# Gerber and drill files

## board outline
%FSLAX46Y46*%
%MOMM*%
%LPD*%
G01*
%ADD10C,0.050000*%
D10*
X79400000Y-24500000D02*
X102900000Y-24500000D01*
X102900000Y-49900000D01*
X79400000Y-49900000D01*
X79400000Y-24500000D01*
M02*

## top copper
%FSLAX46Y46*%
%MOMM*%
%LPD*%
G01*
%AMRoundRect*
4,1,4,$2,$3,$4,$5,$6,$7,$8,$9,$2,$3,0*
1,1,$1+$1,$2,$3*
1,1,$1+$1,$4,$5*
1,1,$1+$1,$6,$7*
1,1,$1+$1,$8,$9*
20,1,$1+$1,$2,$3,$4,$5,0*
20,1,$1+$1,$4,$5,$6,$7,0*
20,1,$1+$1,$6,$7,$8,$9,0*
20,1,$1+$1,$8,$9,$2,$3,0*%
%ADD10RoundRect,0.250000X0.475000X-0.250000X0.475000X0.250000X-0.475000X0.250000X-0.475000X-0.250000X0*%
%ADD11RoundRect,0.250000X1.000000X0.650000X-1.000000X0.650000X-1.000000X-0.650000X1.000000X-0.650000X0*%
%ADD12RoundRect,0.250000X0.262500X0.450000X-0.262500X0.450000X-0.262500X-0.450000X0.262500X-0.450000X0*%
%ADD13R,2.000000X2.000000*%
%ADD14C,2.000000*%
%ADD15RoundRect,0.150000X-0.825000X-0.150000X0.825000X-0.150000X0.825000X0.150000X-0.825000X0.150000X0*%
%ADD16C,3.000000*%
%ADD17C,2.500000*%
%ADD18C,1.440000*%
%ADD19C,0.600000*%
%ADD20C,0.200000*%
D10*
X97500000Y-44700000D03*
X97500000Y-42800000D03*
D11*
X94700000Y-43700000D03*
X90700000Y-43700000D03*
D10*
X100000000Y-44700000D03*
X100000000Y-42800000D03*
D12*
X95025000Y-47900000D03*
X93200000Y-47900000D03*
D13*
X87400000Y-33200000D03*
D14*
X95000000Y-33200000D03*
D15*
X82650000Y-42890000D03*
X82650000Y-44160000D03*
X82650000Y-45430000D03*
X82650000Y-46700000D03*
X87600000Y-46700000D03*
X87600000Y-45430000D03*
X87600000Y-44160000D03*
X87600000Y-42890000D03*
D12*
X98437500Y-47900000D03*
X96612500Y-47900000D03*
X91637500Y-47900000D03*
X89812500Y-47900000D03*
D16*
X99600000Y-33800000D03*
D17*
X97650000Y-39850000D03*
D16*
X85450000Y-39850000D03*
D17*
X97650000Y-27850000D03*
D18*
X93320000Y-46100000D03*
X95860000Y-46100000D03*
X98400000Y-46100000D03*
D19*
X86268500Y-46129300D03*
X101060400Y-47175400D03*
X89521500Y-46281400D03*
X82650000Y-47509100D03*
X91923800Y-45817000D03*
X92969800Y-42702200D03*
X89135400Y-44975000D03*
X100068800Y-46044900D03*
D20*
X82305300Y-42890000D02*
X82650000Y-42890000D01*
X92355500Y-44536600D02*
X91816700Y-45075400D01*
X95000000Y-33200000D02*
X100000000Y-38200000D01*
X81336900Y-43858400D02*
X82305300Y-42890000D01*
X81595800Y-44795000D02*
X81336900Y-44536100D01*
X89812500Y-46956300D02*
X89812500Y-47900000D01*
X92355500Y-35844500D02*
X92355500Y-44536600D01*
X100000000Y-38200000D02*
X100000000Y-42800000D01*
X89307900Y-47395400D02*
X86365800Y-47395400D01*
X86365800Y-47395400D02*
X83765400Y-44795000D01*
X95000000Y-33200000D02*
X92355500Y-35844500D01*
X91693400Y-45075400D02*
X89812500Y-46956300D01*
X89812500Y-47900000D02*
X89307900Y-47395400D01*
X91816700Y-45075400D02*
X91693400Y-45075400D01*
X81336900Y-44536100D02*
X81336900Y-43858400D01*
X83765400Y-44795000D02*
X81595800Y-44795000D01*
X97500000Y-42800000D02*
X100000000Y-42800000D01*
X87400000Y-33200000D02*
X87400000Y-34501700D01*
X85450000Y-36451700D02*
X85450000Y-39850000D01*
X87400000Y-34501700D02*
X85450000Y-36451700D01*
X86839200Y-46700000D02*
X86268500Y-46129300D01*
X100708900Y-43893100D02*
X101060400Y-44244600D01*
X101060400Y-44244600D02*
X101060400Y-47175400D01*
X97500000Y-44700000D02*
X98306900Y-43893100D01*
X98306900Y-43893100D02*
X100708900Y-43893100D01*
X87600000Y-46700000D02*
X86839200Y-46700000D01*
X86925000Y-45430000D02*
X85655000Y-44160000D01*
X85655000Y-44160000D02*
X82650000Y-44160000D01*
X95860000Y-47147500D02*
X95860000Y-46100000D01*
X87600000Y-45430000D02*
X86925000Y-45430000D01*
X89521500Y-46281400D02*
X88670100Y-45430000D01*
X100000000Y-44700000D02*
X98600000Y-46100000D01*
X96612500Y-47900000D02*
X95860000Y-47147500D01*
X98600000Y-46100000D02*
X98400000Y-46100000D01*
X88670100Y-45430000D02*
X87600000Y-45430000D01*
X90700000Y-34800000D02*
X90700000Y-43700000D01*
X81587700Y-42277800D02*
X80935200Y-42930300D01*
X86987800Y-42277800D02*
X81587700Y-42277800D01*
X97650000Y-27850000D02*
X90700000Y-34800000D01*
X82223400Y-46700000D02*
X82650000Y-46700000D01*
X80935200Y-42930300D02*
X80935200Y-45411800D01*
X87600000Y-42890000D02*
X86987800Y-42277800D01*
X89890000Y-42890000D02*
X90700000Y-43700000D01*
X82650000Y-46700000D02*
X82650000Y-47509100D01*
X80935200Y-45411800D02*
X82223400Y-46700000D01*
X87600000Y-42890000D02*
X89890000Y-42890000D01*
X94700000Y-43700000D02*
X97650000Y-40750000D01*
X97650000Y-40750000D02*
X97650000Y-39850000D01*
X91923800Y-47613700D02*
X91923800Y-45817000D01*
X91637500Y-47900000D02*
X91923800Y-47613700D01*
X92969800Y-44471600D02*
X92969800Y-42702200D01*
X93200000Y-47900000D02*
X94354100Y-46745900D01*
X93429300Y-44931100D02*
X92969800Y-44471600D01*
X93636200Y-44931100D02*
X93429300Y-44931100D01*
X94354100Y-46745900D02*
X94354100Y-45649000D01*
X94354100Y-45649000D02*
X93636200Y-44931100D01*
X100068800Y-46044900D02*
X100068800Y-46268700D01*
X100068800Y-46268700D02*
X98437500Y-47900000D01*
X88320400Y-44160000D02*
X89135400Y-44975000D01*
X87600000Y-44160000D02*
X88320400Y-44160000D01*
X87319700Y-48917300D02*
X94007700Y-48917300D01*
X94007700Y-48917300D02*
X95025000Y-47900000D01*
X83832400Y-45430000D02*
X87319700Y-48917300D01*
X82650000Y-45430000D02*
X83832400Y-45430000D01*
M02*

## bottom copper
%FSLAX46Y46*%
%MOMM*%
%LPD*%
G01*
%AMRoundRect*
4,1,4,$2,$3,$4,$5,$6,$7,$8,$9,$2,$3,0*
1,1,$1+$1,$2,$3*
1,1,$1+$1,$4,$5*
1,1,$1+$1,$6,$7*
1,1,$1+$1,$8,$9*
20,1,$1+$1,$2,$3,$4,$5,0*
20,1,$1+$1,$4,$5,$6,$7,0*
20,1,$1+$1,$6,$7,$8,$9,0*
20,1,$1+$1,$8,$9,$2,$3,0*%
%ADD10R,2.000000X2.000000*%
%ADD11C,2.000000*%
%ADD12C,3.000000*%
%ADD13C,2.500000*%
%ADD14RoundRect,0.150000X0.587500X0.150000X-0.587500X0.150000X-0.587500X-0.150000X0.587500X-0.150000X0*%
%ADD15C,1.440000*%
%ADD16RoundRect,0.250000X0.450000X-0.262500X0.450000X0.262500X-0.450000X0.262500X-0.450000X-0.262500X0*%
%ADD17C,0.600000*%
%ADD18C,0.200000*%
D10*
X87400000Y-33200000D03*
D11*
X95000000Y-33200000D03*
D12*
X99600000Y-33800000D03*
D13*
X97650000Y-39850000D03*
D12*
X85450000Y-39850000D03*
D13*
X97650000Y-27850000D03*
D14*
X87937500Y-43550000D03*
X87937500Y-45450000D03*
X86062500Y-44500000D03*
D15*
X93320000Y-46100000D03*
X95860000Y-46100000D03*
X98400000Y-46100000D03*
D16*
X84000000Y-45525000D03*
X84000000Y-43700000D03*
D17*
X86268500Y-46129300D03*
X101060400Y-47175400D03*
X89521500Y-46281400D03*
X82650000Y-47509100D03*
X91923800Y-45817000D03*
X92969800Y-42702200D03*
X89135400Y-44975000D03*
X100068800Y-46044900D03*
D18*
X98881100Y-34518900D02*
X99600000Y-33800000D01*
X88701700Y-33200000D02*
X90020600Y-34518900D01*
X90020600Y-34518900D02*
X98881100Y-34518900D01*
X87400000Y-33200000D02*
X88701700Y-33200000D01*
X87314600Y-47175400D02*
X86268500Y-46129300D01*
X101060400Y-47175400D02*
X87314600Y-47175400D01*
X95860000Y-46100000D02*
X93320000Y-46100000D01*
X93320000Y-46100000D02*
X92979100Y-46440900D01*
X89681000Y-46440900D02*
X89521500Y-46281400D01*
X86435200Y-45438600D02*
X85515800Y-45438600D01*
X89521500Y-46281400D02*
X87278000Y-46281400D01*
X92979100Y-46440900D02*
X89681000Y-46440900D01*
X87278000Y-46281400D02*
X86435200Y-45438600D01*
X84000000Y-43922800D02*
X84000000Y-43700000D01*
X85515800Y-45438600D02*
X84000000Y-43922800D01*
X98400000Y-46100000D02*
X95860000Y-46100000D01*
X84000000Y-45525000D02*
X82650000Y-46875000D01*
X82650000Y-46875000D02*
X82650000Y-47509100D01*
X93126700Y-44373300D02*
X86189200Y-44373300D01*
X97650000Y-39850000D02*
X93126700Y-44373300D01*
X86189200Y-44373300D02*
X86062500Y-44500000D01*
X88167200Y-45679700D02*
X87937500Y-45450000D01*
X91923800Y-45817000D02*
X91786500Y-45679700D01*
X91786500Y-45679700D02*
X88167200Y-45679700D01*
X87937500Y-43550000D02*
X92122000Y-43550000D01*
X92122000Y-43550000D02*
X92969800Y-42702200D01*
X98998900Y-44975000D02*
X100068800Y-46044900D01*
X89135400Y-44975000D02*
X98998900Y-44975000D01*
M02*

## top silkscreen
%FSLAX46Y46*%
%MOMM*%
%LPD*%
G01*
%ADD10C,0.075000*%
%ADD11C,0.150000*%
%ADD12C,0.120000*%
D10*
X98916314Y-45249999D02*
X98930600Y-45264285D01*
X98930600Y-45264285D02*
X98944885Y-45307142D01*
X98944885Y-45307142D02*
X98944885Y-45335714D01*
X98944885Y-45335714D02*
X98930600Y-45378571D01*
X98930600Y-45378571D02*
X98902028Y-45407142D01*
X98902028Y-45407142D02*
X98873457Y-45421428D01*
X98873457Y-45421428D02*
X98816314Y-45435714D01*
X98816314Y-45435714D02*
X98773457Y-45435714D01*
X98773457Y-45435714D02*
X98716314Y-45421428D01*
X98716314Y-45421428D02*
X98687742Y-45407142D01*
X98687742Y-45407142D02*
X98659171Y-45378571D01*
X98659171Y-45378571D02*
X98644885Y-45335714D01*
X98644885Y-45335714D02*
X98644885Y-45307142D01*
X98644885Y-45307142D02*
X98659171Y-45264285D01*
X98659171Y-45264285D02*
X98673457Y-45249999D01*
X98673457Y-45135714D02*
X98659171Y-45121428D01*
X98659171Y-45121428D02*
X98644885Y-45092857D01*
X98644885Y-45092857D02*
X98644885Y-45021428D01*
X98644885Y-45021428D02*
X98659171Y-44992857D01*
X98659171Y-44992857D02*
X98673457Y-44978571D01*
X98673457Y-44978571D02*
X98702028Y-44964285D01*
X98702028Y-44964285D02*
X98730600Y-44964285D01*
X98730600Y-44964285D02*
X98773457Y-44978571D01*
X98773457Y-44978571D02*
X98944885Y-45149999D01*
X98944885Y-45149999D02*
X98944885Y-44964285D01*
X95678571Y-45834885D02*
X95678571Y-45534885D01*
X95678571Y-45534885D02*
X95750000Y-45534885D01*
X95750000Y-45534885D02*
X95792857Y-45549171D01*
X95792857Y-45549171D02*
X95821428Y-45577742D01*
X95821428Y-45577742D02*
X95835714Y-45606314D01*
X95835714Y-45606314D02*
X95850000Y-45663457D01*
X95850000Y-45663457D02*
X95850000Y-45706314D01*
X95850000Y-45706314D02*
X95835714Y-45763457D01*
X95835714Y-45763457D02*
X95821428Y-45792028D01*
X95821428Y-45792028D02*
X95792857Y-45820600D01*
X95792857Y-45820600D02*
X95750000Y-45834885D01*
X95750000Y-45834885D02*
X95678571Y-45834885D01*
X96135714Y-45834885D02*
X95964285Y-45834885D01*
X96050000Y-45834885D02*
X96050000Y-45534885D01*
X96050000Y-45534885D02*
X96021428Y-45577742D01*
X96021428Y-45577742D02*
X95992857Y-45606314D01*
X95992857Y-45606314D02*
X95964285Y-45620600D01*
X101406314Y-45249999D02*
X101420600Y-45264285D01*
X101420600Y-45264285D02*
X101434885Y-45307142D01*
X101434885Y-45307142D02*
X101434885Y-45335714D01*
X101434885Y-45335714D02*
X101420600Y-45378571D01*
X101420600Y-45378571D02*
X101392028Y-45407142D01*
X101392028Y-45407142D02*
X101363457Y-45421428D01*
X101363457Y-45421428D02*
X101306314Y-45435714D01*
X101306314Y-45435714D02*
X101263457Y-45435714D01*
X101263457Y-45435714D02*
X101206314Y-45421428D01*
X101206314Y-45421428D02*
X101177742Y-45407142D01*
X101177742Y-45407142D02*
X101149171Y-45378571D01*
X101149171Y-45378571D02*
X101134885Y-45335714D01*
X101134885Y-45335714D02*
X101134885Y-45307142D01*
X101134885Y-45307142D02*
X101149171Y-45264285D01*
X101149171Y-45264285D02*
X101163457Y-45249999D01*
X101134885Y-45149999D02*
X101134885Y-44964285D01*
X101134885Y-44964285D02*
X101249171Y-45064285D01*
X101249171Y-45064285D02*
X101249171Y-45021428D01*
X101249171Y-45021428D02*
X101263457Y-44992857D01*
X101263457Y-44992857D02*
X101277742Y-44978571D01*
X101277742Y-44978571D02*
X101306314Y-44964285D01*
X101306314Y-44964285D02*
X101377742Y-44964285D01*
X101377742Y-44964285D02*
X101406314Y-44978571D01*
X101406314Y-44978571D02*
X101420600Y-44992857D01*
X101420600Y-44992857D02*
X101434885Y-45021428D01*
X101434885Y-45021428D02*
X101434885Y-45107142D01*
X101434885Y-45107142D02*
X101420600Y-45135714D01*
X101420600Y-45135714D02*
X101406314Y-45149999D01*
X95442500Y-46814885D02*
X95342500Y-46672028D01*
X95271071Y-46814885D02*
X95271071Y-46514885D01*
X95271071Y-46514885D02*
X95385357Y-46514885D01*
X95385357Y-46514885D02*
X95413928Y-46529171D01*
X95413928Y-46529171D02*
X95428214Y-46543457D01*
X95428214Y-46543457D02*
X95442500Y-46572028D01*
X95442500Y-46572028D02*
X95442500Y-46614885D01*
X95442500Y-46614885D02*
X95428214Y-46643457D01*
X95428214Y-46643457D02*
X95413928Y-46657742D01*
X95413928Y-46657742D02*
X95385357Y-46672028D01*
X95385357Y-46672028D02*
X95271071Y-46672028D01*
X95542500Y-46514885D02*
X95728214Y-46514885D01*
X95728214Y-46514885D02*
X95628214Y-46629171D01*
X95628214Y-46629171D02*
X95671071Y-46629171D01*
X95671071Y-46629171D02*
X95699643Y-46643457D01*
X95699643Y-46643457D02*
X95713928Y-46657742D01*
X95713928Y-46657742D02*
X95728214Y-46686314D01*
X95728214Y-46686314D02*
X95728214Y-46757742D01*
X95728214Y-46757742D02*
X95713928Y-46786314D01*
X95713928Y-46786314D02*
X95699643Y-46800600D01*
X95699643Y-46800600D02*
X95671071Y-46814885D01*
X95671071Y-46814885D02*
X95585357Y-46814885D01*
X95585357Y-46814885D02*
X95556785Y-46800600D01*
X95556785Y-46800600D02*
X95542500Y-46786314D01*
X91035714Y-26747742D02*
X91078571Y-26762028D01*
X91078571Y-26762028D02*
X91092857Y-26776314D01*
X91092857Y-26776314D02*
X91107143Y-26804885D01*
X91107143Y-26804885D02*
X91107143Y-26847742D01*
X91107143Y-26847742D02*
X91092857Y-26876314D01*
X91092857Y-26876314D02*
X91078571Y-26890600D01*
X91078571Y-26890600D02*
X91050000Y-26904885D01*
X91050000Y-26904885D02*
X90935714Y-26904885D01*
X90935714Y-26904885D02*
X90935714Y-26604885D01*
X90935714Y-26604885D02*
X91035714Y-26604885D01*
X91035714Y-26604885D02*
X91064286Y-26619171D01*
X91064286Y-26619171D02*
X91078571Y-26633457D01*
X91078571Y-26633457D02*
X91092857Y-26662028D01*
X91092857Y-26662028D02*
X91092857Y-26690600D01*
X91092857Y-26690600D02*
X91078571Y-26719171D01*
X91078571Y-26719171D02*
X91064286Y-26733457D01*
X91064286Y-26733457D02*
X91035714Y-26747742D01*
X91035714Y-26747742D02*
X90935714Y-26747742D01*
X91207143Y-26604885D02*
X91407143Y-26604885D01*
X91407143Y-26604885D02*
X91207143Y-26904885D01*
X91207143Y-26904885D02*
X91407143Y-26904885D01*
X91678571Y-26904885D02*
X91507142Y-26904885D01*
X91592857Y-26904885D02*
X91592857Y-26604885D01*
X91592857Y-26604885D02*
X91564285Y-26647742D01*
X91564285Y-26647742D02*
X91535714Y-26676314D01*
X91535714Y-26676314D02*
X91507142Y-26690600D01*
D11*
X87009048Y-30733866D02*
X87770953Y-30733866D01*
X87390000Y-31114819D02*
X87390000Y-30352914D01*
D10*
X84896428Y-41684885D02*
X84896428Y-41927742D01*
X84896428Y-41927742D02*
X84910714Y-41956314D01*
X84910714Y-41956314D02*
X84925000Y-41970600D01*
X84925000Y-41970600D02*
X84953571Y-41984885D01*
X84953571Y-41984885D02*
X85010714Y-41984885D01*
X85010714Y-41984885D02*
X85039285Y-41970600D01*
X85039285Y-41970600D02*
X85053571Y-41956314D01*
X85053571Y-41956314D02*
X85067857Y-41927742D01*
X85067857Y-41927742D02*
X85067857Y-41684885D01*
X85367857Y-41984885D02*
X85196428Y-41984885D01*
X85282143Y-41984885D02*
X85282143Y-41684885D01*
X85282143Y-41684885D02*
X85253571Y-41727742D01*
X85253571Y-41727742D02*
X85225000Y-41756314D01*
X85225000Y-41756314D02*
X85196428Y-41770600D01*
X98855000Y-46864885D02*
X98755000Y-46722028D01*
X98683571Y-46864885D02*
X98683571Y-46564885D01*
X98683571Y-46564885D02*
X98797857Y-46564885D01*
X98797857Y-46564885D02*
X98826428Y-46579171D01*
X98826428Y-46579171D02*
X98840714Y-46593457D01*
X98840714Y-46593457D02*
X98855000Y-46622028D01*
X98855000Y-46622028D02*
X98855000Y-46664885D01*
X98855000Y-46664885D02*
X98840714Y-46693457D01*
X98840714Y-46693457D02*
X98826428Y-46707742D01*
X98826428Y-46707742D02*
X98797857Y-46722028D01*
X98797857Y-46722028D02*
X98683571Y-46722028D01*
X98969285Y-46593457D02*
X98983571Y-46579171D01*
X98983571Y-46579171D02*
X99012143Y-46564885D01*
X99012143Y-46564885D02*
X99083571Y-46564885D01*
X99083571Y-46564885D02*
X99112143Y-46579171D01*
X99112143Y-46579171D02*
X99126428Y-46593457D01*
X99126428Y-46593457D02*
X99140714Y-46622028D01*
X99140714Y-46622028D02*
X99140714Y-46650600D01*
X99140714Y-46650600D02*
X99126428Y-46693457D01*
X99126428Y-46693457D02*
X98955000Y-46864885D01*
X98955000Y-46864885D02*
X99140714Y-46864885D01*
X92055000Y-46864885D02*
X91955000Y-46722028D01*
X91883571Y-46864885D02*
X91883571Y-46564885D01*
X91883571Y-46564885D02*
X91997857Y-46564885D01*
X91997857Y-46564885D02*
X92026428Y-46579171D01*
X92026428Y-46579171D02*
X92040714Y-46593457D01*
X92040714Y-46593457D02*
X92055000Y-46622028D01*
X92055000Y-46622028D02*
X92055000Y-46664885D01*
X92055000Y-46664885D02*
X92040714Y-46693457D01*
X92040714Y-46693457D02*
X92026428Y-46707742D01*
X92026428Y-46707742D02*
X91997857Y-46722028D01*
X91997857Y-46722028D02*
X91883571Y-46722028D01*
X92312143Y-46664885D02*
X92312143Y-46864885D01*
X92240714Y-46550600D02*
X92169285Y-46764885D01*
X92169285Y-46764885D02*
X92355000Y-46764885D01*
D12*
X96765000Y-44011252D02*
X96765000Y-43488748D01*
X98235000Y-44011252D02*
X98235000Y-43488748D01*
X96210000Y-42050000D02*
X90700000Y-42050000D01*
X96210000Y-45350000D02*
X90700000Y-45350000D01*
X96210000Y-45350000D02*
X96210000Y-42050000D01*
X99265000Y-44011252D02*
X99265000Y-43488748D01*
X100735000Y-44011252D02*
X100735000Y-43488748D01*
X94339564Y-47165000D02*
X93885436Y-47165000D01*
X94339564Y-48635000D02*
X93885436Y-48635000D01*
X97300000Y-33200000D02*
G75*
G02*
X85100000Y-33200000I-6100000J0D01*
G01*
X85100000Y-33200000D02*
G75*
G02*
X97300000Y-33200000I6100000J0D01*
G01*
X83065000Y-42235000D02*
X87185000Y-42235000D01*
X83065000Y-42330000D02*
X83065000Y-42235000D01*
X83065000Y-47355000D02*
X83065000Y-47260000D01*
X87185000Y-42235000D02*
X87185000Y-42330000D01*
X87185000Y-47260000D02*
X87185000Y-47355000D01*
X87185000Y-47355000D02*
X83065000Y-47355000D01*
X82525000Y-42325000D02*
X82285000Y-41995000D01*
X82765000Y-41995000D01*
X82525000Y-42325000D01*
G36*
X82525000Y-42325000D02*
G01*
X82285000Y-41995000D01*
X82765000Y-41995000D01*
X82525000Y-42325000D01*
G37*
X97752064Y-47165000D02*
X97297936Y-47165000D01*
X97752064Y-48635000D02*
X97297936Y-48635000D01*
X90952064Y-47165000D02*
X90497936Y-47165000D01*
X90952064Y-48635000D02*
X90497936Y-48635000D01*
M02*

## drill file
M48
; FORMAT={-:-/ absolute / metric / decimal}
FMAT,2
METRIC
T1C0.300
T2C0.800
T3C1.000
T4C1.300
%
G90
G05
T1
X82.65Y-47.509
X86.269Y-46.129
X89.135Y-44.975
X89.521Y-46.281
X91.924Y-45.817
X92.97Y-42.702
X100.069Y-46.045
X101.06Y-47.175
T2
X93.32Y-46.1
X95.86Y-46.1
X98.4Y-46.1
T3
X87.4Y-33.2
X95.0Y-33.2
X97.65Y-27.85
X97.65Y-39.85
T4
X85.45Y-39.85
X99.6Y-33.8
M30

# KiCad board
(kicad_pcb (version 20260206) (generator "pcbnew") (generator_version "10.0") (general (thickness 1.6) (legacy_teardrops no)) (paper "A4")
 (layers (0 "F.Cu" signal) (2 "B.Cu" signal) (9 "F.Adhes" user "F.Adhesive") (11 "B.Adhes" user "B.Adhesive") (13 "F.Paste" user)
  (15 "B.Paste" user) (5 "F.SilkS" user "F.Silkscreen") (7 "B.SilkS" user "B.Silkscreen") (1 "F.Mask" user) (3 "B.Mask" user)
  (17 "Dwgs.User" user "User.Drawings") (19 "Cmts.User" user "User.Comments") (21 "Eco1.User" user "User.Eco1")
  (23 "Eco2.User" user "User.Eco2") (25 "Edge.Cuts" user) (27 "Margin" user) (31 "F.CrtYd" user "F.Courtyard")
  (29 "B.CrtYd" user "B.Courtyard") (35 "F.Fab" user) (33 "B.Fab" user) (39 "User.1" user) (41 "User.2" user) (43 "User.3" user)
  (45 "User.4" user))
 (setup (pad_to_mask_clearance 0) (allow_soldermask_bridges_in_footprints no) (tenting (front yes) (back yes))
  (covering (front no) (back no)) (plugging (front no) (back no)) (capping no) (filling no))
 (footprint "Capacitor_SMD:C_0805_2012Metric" (layer "F.Cu") (at 97.5 43.75 90)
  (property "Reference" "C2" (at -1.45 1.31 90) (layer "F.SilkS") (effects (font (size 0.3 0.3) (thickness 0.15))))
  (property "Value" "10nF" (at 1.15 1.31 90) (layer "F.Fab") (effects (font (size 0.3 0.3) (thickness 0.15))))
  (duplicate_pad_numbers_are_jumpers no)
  (fp_line (start -0.261252 -0.735) (end 0.261252 -0.735) (stroke (width 0.12) (type solid)) (layer "F.SilkS"))
  (fp_line (start -0.261252 0.735) (end 0.261252 0.735) (stroke (width 0.12) (type solid)) (layer "F.SilkS"))
  (pad "1" smd roundrect (at -0.95 0 90) (size 1 1.45) (layers "F.Cu" "F.Mask" "F.Paste") (roundrect_rratio 0.25) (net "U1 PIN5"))
  (pad "2" smd roundrect (at 0.95 0 90) (size 1 1.45) (layers "F.Cu" "F.Mask" "F.Paste") (roundrect_rratio 0.25) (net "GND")))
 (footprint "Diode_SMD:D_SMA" (layer "F.Cu") (at 92.7 43.7 180)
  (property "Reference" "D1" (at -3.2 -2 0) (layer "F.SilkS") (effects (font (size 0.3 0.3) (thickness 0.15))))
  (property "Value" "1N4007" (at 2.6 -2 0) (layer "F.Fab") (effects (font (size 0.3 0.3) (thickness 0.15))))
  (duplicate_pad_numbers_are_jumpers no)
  (fp_line (start -3.51 1.65) (end 2 1.65) (stroke (width 0.12) (type solid)) (layer "F.SilkS"))
  (fp_line (start -3.51 -1.65) (end 2 -1.65) (stroke (width 0.12) (type solid)) (layer "F.SilkS"))
  (fp_line (start -3.51 -1.65) (end -3.51 1.65) (stroke (width 0.12) (type solid)) (layer "F.SilkS"))
  (pad "1" smd roundrect (at -2 0 180) (size 2.5 1.8) (layers "F.Cu" "F.Mask" "F.Paste") (roundrect_rratio 0.1388888889) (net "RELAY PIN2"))
  (pad "2" smd roundrect (at 2 0 180) (size 2.5 1.8) (layers "F.Cu" "F.Mask" "F.Paste") (roundrect_rratio 0.1388888889) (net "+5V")))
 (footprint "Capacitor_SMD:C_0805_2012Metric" (layer "F.Cu") (at 100 43.75 90)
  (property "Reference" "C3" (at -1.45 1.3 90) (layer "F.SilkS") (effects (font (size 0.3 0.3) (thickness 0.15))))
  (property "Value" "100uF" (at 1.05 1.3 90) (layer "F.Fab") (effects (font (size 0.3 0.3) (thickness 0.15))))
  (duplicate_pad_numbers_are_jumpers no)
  (fp_line (start -0.261252 -0.735) (end 0.261252 -0.735) (stroke (width 0.12) (type solid)) (layer "F.SilkS"))
  (fp_line (start -0.261252 0.735) (end 0.261252 0.735) (stroke (width 0.12) (type solid)) (layer "F.SilkS"))
  (pad "1" smd roundrect (at -0.95 0 90) (size 1 1.45) (layers "F.Cu" "F.Mask" "F.Paste") (roundrect_rratio 0.25) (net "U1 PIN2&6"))
  (pad "2" smd roundrect (at 0.95 0 90) (size 1 1.45) (layers "F.Cu" "F.Mask" "F.Paste") (roundrect_rratio 0.25) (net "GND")))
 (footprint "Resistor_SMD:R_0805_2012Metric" (layer "F.Cu") (at 94.1125 47.9 180)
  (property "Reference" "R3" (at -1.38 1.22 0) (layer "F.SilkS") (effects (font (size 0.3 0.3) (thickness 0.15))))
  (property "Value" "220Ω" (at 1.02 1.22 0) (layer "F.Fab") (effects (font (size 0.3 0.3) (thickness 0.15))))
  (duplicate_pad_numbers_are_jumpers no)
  (fp_line (start -0.227064 0.735) (end 0.227064 0.735) (stroke (width 0.12) (type solid)) (layer "F.SilkS"))
  (fp_line (start -0.227064 -0.735) (end 0.227064 -0.735) (stroke (width 0.12) (type solid)) (layer "F.SilkS"))
  (pad "1" smd roundrect (at -0.9125 0 180) (size 1.025 1.4) (layers "F.Cu" "F.Mask" "F.Paste") (roundrect_rratio 0.243902) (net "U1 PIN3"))
  (pad "2" smd roundrect (at 0.9125 0 180) (size 1.025 1.4) (layers "F.Cu" "F.Mask" "F.Paste") (roundrect_rratio 0.243902)
   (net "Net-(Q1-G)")))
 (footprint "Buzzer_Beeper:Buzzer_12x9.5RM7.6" (layer "F.Cu") (at 87.4 33.2)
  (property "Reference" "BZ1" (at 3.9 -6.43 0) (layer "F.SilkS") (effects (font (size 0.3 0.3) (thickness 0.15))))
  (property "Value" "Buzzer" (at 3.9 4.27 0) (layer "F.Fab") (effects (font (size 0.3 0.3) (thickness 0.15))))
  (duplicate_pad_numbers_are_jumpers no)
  (fp_circle (center 3.8 0) (end 9.9 0) (stroke (width 0.12) (type solid)) (fill no) (layer "F.SilkS"))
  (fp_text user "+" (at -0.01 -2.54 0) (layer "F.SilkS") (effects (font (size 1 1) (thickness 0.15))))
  (pad "1" thru_hole rect (at 0 0) (size 2 2) (drill 1) (layers "*.Cu" "*.Mask") (remove_unused_layers no) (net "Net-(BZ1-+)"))
  (pad "2" thru_hole circle (at 7.6 0) (size 2 2) (drill 1) (layers "*.Cu" "*.Mask") (remove_unused_layers no) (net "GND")))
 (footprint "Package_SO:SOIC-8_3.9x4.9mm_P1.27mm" (layer "F.Cu") (at 85.125 44.795)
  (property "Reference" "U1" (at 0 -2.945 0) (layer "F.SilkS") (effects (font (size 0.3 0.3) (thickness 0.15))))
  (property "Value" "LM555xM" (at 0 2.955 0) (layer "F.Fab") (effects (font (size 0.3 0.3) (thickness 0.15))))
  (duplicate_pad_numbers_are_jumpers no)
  (fp_line (start -2.06 -2.56) (end 2.06 -2.56) (stroke (width 0.12) (type solid)) (layer "F.SilkS"))
  (fp_line (start -2.06 -2.465) (end -2.06 -2.56) (stroke (width 0.12) (type solid)) (layer "F.SilkS"))
  (fp_line (start -2.06 2.56) (end -2.06 2.465) (stroke (width 0.12) (type solid)) (layer "F.SilkS"))
  (fp_line (start 2.06 -2.56) (end 2.06 -2.465) (stroke (width 0.12) (type solid)) (layer "F.SilkS"))
  (fp_line (start 2.06 2.465) (end 2.06 2.56) (stroke (width 0.12) (type solid)) (layer "F.SilkS"))
  (fp_line (start 2.06 2.56) (end -2.06 2.56) (stroke (width 0.12) (type solid)) (layer "F.SilkS"))
  (fp_poly (pts (xy -2.6 -2.47) (xy -2.84 -2.8) (xy -2.36 -2.8)) (stroke (width 0.12) (type solid)) (fill yes) (layer "F.SilkS"))
  (pad "1" smd roundrect (at -2.475 -1.905) (size 1.95 0.6) (layers "F.Cu" "F.Mask" "F.Paste") (roundrect_rratio 0.25) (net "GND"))
  (pad "2" smd roundrect (at -2.475 -0.635) (size 1.95 0.6) (layers "F.Cu" "F.Mask" "F.Paste") (roundrect_rratio 0.25) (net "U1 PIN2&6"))
  (pad "3" smd roundrect (at -2.475 0.635) (size 1.95 0.6) (layers "F.Cu" "F.Mask" "F.Paste") (roundrect_rratio 0.25) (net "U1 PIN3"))
  (pad "4" smd roundrect (at -2.475 1.905) (size 1.95 0.6) (layers "F.Cu" "F.Mask" "F.Paste") (roundrect_rratio 0.25) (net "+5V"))
  (pad "5" smd roundrect (at 2.475 1.905) (size 1.95 0.6) (layers "F.Cu" "F.Mask" "F.Paste") (roundrect_rratio 0.25) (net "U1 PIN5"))
  (pad "6" smd roundrect (at 2.475 0.635) (size 1.95 0.6) (layers "F.Cu" "F.Mask" "F.Paste") (roundrect_rratio 0.25) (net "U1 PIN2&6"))
  (pad "7" smd roundrect (at 2.475 -0.635) (size 1.95 0.6) (layers "F.Cu" "F.Mask" "F.Paste") (roundrect_rratio 0.25) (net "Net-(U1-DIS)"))
  (pad "8" smd roundrect (at 2.475 -1.905) (size 1.95 0.6) (layers "F.Cu" "F.Mask" "F.Paste") (roundrect_rratio 0.25) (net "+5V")))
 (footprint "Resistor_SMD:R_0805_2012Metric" (layer "F.Cu") (at 97.525 47.9 180)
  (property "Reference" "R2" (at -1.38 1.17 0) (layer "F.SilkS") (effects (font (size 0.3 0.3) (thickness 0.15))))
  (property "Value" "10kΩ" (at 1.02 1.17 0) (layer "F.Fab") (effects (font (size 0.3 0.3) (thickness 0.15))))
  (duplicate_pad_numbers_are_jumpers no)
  (fp_line (start -0.227064 0.735) (end 0.227064 0.735) (stroke (width 0.12) (type solid)) (layer "F.SilkS"))
  (fp_line (start -0.227064 -0.735) (end 0.227064 -0.735) (stroke (width 0.12) (type solid)) (layer "F.SilkS"))
  (pad "1" smd roundrect (at -0.9125 0 180) (size 1.025 1.4) (layers "F.Cu" "F.Mask" "F.Paste") (roundrect_rratio 0.243902)
   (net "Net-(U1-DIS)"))
  (pad "2" smd roundrect (at 0.9125 0 180) (size 1.025 1.4) (layers "F.Cu" "F.Mask" "F.Paste") (roundrect_rratio 0.243902) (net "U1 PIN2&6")))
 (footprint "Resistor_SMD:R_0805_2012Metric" (layer "F.Cu") (at 90.725 47.9 180)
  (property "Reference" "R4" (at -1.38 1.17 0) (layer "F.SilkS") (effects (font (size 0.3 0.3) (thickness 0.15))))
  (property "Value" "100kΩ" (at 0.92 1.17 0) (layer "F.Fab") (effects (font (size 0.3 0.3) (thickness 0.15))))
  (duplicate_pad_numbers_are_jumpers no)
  (fp_line (start -0.227064 0.735) (end 0.227064 0.735) (stroke (width 0.12) (type solid)) (layer "F.SilkS"))
  (fp_line (start -0.227064 -0.735) (end 0.227064 -0.735) (stroke (width 0.12) (type solid)) (layer "F.SilkS"))
  (pad "1" smd roundrect (at -0.9125 0 180) (size 1.025 1.4) (layers "F.Cu" "F.Mask" "F.Paste") (roundrect_rratio 0.243902)
   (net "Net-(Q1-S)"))
  (pad "2" smd roundrect (at 0.9125 0 180) (size 1.025 1.4) (layers "F.Cu" "F.Mask" "F.Paste") (roundrect_rratio 0.243902) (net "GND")))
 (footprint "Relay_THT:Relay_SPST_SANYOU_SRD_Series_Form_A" (layer "B.Cu") (at 99.6 33.8 180)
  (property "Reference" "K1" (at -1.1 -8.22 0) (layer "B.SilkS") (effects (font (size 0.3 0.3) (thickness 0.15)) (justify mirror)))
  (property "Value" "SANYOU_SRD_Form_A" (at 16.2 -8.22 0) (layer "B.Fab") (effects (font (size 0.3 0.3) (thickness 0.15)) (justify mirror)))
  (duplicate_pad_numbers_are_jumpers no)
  (pad "1" thru_hole circle (at 0 0 90) (size 3 3) (drill 1.3) (layers "*.Cu" "*.Mask") (remove_unused_layers no) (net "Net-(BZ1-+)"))
  (pad "2" thru_hole circle (at 1.95 -6.05 90) (size 2.5 2.5) (drill 1) (layers "*.Cu" "*.Mask") (remove_unused_layers no)
   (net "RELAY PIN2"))
  (pad "3" thru_hole circle (at 14.15 -6.05 90) (size 3 3) (drill 1.3) (layers "*.Cu" "*.Mask") (remove_unused_layers no)
   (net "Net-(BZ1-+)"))
  (pad "5" thru_hole circle (at 1.95 5.95 90) (size 2.5 2.5) (drill 1) (layers "*.Cu" "*.Mask") (remove_unused_layers no) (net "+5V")))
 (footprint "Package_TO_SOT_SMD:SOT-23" (layer "B.Cu") (at 87 44.5 180)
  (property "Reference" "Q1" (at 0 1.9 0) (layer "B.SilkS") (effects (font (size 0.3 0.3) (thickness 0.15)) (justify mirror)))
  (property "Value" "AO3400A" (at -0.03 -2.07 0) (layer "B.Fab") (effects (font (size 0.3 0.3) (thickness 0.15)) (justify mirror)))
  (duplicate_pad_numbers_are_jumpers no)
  (pad "1" smd roundrect (at -0.9375 0.95 180) (size 1.475 0.6) (layers "B.Cu" "B.Mask" "B.Paste") (roundrect_rratio 0.25)
   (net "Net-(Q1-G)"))
  (pad "2" smd roundrect (at -0.9375 -0.95 180) (size 1.475 0.6) (layers "B.Cu" "B.Mask" "B.Paste") (roundrect_rratio 0.25)
   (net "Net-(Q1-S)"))
  (pad "3" smd roundrect (at 0.9375 0 180) (size 1.475 0.6) (layers "B.Cu" "B.Mask" "B.Paste") (roundrect_rratio 0.25) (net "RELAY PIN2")))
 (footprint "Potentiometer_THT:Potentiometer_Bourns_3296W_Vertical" (layer "B.Cu") (at 93.32 46.1 180)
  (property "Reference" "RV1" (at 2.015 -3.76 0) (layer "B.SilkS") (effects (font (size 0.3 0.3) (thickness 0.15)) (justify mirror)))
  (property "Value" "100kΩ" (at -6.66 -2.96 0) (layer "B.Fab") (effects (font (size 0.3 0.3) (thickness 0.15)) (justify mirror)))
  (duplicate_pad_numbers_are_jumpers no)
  (pad "1" thru_hole circle (at 0 0 180) (size 1.44 1.44) (drill 0.8) (layers "*.Cu" "*.Mask") (remove_unused_layers no) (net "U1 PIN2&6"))
  (pad "2" thru_hole circle (at -2.54 0 180) (size 1.44 1.44) (drill 0.8) (layers "*.Cu" "*.Mask") (remove_unused_layers no)
   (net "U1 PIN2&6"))
  (pad "3" thru_hole circle (at -5.08 0 180) (size 1.44 1.44) (drill 0.8) (layers "*.Cu" "*.Mask") (remove_unused_layers no)
   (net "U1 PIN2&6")))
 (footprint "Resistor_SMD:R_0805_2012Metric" (layer "B.Cu") (at 84 44.6125 90)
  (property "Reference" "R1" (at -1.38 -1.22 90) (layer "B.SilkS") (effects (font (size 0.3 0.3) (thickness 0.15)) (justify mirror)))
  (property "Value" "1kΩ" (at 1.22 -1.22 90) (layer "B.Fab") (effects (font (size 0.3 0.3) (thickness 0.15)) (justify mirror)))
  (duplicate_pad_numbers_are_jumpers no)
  (pad "1" smd roundrect (at -0.9125 0 90) (size 1.025 1.4) (layers "B.Cu" "B.Mask" "B.Paste") (roundrect_rratio 0.243902) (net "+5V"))
  (pad "2" smd roundrect (at 0.9125 0 90) (size 1.025 1.4) (layers "B.Cu" "B.Mask" "B.Paste") (roundrect_rratio 0.243902) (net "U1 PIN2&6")))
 (gr_rect (start 79.4 24.5) (end 102.9 49.9) (stroke (width 0.05) (type default)) (fill no) (layer "Edge.Cuts"))
 (segment (start 82.3053 42.89) (end 82.65 42.89) (width 0.2) (layer "F.Cu") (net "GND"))
 (segment (start 92.3555 44.5366) (end 91.8167 45.0754) (width 0.2) (layer "F.Cu") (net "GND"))
 (segment (start 95 33.2) (end 100 38.2) (width 0.2) (layer "F.Cu") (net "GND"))
 (segment (start 81.3369 43.8584) (end 82.3053 42.89) (width 0.2) (layer "F.Cu") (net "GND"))
 (segment (start 81.5958 44.795) (end 81.3369 44.5361) (width 0.2) (layer "F.Cu") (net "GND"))
 (segment (start 89.8125 46.9563) (end 89.8125 47.9) (width 0.2) (layer "F.Cu") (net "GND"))
 (segment (start 92.3555 35.8445) (end 92.3555 44.5366) (width 0.2) (layer "F.Cu") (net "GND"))
 (segment (start 100 38.2) (end 100 42.8) (width 0.2) (layer "F.Cu") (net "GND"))
 (segment (start 89.3079 47.3954) (end 86.3658 47.3954) (width 0.2) (layer "F.Cu") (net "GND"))
 (segment (start 86.3658 47.3954) (end 83.7654 44.795) (width 0.2) (layer "F.Cu") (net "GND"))
 (segment (start 95 33.2) (end 92.3555 35.8445) (width 0.2) (layer "F.Cu") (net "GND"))
 (segment (start 91.6934 45.0754) (end 89.8125 46.9563) (width 0.2) (layer "F.Cu") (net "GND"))
 (segment (start 89.8125 47.9) (end 89.3079 47.3954) (width 0.2) (layer "F.Cu") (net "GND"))
 (segment (start 91.8167 45.0754) (end 91.6934 45.0754) (width 0.2) (layer "F.Cu") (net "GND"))
 (segment (start 81.3369 44.5361) (end 81.3369 43.8584) (width 0.2) (layer "F.Cu") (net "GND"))
 (segment (start 83.7654 44.795) (end 81.5958 44.795) (width 0.2) (layer "F.Cu") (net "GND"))
 (segment (start 97.5 42.8) (end 100 42.8) (width 0.2) (layer "F.Cu") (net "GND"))
 (segment (start 87.4 33.2) (end 87.4 34.5017) (width 0.2) (layer "F.Cu") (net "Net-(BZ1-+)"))
 (segment (start 85.45 36.4517) (end 85.45 39.85) (width 0.2) (layer "F.Cu") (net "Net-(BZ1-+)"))
 (segment (start 87.4 34.5017) (end 85.45 36.4517) (width 0.2) (layer "F.Cu") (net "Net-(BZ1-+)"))
 (segment (start 98.8811 34.5189) (end 99.6 33.8) (width 0.2) (layer "B.Cu") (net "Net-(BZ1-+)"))
 (segment (start 88.7017 33.2) (end 90.0206 34.5189) (width 0.2) (layer "B.Cu") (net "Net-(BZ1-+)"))
 (segment (start 90.0206 34.5189) (end 98.8811 34.5189) (width 0.2) (layer "B.Cu") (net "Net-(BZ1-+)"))
 (segment (start 87.4 33.2) (end 88.7017 33.2) (width 0.2) (layer "B.Cu") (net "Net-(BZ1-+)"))
 (segment (start 86.8392 46.7) (end 86.2685 46.1293) (width 0.2) (layer "F.Cu") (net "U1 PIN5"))
 (segment (start 100.7089 43.8931) (end 101.0604 44.2446) (width 0.2) (layer "F.Cu") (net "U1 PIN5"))
 (segment (start 101.0604 44.2446) (end 101.0604 47.1754) (width 0.2) (layer "F.Cu") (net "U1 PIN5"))
 (segment (start 97.5 44.7) (end 98.3069 43.8931) (width 0.2) (layer "F.Cu") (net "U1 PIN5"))
 (segment (start 98.3069 43.8931) (end 100.7089 43.8931) (width 0.2) (layer "F.Cu") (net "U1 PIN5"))
 (segment (start 87.6 46.7) (end 86.8392 46.7) (width 0.2) (layer "F.Cu") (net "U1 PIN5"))
 (via (at 86.2685 46.1293) (size 0.6) (drill 0.3) (layers "F.Cu" "B.Cu") (capping no) (covering (front no) (back no))
  (plugging (front no) (back no)) (filling no) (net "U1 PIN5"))
 (via (at 101.0604 47.1754) (size 0.6) (drill 0.3) (layers "F.Cu" "B.Cu") (capping no) (covering (front no) (back no))
  (plugging (front no) (back no)) (filling no) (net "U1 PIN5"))
 (segment (start 87.3146 47.1754) (end 86.2685 46.1293) (width 0.2) (layer "B.Cu") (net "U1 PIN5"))
 (segment (start 101.0604 47.1754) (end 87.3146 47.1754) (width 0.2) (layer "B.Cu") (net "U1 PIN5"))
 (segment (start 86.925 45.43) (end 85.655 44.16) (width 0.2) (layer "F.Cu") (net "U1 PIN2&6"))
 (segment (start 85.655 44.16) (end 82.65 44.16) (width 0.2) (layer "F.Cu") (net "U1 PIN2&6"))
 (segment (start 95.86 47.1475) (end 95.86 46.1) (width 0.2) (layer "F.Cu") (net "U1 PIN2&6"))
 (segment (start 87.6 45.43) (end 86.925 45.43) (width 0.2) (layer "F.Cu") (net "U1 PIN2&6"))
 (segment (start 89.5215 46.2814) (end 88.6701 45.43) (width 0.2) (layer "F.Cu") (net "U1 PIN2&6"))
 (segment (start 100 44.7) (end 98.6 46.1) (width 0.2) (layer "F.Cu") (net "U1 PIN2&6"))
 (segment (start 96.6125 47.9) (end 95.86 47.1475) (width 0.2) (layer "F.Cu") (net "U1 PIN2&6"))
 (segment (start 98.6 46.1) (end 98.4 46.1) (width 0.2) (layer "F.Cu") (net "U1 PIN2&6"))
 (segment (start 88.6701 45.43) (end 87.6 45.43) (width 0.2) (layer "F.Cu") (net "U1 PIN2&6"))
 (via (at 89.5215 46.2814) (size 0.6) (drill 0.3) (layers "F.Cu" "B.Cu") (capping no) (covering (front no) (back no))
  (plugging (front no) (back no)) (filling no) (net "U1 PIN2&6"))
 (segment (start 95.86 46.1) (end 93.32 46.1) (width 0.2) (layer "B.Cu") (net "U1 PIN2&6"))
 (segment (start 93.32 46.1) (end 92.9791 46.4409) (width 0.2) (layer "B.Cu") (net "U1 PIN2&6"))
 (segment (start 89.681 46.4409) (end 89.5215 46.2814) (width 0.2) (layer "B.Cu") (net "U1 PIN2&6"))
 (segment (start 86.4352 45.4386) (end 85.5158 45.4386) (width 0.2) (layer "B.Cu") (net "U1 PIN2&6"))
 (segment (start 89.5215 46.2814) (end 87.278 46.2814) (width 0.2) (layer "B.Cu") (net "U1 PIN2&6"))
 (segment (start 92.9791 46.4409) (end 89.681 46.4409) (width 0.2) (layer "B.Cu") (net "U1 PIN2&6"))
 (segment (start 87.278 46.2814) (end 86.4352 45.4386) (width 0.2) (layer "B.Cu") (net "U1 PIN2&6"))
 (segment (start 84 43.9228) (end 84 43.7) (width 0.2) (layer "B.Cu") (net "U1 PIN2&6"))
 (segment (start 85.5158 45.4386) (end 84 43.9228) (width 0.2) (layer "B.Cu") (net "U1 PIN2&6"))
 (segment (start 98.4 46.1) (end 95.86 46.1) (width 0.2) (layer "B.Cu") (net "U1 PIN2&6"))
 (segment (start 90.7 34.8) (end 90.7 43.7) (width 0.2) (layer "F.Cu") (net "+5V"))
 (segment (start 81.5877 42.2778) (end 80.9352 42.9303) (width 0.2) (layer "F.Cu") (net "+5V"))
 (segment (start 86.9878 42.2778) (end 81.5877 42.2778) (width 0.2) (layer "F.Cu") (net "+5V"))
 (segment (start 97.65 27.85) (end 90.7 34.8) (width 0.2) (layer "F.Cu") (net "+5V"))
 (segment (start 82.2234 46.7) (end 82.65 46.7) (width 0.2) (layer "F.Cu") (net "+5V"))
 (segment (start 80.9352 42.9303) (end 80.9352 45.4118) (width 0.2) (layer "F.Cu") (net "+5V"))
 (segment (start 87.6 42.89) (end 86.9878 42.2778) (width 0.2) (layer "F.Cu") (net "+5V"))
 (segment (start 89.89 42.89) (end 90.7 43.7) (width 0.2) (layer "F.Cu") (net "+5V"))
 (segment (start 82.65 46.7) (end 82.65 47.5091) (width 0.2) (layer "F.Cu") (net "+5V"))
 (segment (start 80.9352 45.4118) (end 82.2234 46.7) (width 0.2) (layer "F.Cu") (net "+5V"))
 (segment (start 87.6 42.89) (end 89.89 42.89) (width 0.2) (layer "F.Cu") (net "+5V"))
 (via (at 82.65 47.5091) (size 0.6) (drill 0.3) (layers "F.Cu" "B.Cu") (capping no) (covering (front no) (back no))
  (plugging (front no) (back no)) (filling no) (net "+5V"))
 (segment (start 84 45.525) (end 82.65 46.875) (width 0.2) (layer "B.Cu") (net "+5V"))
 (segment (start 82.65 46.875) (end 82.65 47.5091) (width 0.2) (layer "B.Cu") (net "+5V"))
 (segment (start 94.7 43.7) (end 97.65 40.75) (width 0.2) (layer "F.Cu") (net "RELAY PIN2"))
 (segment (start 97.65 40.75) (end 97.65 39.85) (width 0.2) (layer "F.Cu") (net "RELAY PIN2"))
 (segment (start 93.1267 44.3733) (end 86.1892 44.3733) (width 0.2) (layer "B.Cu") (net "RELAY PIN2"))
 (segment (start 97.65 39.85) (end 93.1267 44.3733) (width 0.2) (layer "B.Cu") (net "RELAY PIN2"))
 (segment (start 86.1892 44.3733) (end 86.0625 44.5) (width 0.2) (layer "B.Cu") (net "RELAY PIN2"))
 (segment (start 91.9238 47.6137) (end 91.9238 45.817) (width 0.2) (layer "F.Cu") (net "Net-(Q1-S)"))
 (segment (start 91.6375 47.9) (end 91.9238 47.6137) (width 0.2) (layer "F.Cu") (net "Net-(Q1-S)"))
 (via (at 91.9238 45.817) (size 0.6) (drill 0.3) (layers "F.Cu" "B.Cu") (capping no) (covering (front no) (back no))
  (plugging (front no) (back no)) (filling no) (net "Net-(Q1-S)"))
 (segment (start 88.1672 45.6797) (end 87.9375 45.45) (width 0.2) (layer "B.Cu") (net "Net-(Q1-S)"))
 (segment (start 91.9238 45.817) (end 91.7865 45.6797) (width 0.2) (layer "B.Cu") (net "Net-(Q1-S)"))
 (segment (start 91.7865 45.6797) (end 88.1672 45.6797) (width 0.2) (layer "B.Cu") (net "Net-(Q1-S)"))
 (segment (start 92.9698 44.4716) (end 92.9698 42.7022) (width 0.2) (layer "F.Cu") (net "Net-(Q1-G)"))
 (segment (start 93.2 47.9) (end 94.3541 46.7459) (width 0.2) (layer "F.Cu") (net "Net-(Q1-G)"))
 (segment (start 93.4293 44.9311) (end 92.9698 44.4716) (width 0.2) (layer "F.Cu") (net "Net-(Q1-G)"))
 (segment (start 93.6362 44.9311) (end 93.4293 44.9311) (width 0.2) (layer "F.Cu") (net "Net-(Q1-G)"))
 (segment (start 94.3541 46.7459) (end 94.3541 45.649) (width 0.2) (layer "F.Cu") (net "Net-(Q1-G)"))
 (segment (start 94.3541 45.649) (end 93.6362 44.9311) (width 0.2) (layer "F.Cu") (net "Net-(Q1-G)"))
 (via (at 92.9698 42.7022) (size 0.6) (drill 0.3) (layers "F.Cu" "B.Cu") (capping no) (covering (front no) (back no))
  (plugging (front no) (back no)) (filling no) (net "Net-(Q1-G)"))
 (segment (start 87.9375 43.55) (end 92.122 43.55) (width 0.2) (layer "B.Cu") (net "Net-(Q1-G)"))
 (segment (start 92.122 43.55) (end 92.9698 42.7022) (width 0.2) (layer "B.Cu") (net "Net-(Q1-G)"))
 (segment (start 100.0688 46.0449) (end 100.0688 46.2687) (width 0.2) (layer "F.Cu") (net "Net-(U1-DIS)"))
 (segment (start 100.0688 46.2687) (end 98.4375 47.9) (width 0.2) (layer "F.Cu") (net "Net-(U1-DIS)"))
 (segment (start 88.3204 44.16) (end 89.1354 44.975) (width 0.2) (layer "F.Cu") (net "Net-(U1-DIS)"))
 (segment (start 87.6 44.16) (end 88.3204 44.16) (width 0.2) (layer "F.Cu") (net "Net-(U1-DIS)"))
 (via (at 89.1354 44.975) (size 0.6) (drill 0.3) (layers "F.Cu" "B.Cu") (capping no) (covering (front no) (back no))
  (plugging (front no) (back no)) (filling no) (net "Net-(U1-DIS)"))
 (via (at 100.0688 46.0449) (size 0.6) (drill 0.3) (layers "F.Cu" "B.Cu") (capping no) (covering (front no) (back no))
  (plugging (front no) (back no)) (filling no) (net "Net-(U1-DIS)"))
 (segment (start 98.9989 44.975) (end 100.0688 46.0449) (width 0.2) (layer "B.Cu") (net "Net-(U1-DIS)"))
 (segment (start 89.1354 44.975) (end 98.9989 44.975) (width 0.2) (layer "B.Cu") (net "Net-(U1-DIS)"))
 (segment (start 87.3197 48.9173) (end 94.0077 48.9173) (width 0.2) (layer "F.Cu") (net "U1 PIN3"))
 (segment (start 94.0077 48.9173) (end 95.025 47.9) (width 0.2) (layer "F.Cu") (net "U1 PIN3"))
 (segment (start 83.8324 45.43) (end 87.3197 48.9173) (width 0.2) (layer "F.Cu") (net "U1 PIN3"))
 (segment (start 82.65 45.43) (end 83.8324 45.43) (width 0.2) (layer "F.Cu") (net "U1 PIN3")))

